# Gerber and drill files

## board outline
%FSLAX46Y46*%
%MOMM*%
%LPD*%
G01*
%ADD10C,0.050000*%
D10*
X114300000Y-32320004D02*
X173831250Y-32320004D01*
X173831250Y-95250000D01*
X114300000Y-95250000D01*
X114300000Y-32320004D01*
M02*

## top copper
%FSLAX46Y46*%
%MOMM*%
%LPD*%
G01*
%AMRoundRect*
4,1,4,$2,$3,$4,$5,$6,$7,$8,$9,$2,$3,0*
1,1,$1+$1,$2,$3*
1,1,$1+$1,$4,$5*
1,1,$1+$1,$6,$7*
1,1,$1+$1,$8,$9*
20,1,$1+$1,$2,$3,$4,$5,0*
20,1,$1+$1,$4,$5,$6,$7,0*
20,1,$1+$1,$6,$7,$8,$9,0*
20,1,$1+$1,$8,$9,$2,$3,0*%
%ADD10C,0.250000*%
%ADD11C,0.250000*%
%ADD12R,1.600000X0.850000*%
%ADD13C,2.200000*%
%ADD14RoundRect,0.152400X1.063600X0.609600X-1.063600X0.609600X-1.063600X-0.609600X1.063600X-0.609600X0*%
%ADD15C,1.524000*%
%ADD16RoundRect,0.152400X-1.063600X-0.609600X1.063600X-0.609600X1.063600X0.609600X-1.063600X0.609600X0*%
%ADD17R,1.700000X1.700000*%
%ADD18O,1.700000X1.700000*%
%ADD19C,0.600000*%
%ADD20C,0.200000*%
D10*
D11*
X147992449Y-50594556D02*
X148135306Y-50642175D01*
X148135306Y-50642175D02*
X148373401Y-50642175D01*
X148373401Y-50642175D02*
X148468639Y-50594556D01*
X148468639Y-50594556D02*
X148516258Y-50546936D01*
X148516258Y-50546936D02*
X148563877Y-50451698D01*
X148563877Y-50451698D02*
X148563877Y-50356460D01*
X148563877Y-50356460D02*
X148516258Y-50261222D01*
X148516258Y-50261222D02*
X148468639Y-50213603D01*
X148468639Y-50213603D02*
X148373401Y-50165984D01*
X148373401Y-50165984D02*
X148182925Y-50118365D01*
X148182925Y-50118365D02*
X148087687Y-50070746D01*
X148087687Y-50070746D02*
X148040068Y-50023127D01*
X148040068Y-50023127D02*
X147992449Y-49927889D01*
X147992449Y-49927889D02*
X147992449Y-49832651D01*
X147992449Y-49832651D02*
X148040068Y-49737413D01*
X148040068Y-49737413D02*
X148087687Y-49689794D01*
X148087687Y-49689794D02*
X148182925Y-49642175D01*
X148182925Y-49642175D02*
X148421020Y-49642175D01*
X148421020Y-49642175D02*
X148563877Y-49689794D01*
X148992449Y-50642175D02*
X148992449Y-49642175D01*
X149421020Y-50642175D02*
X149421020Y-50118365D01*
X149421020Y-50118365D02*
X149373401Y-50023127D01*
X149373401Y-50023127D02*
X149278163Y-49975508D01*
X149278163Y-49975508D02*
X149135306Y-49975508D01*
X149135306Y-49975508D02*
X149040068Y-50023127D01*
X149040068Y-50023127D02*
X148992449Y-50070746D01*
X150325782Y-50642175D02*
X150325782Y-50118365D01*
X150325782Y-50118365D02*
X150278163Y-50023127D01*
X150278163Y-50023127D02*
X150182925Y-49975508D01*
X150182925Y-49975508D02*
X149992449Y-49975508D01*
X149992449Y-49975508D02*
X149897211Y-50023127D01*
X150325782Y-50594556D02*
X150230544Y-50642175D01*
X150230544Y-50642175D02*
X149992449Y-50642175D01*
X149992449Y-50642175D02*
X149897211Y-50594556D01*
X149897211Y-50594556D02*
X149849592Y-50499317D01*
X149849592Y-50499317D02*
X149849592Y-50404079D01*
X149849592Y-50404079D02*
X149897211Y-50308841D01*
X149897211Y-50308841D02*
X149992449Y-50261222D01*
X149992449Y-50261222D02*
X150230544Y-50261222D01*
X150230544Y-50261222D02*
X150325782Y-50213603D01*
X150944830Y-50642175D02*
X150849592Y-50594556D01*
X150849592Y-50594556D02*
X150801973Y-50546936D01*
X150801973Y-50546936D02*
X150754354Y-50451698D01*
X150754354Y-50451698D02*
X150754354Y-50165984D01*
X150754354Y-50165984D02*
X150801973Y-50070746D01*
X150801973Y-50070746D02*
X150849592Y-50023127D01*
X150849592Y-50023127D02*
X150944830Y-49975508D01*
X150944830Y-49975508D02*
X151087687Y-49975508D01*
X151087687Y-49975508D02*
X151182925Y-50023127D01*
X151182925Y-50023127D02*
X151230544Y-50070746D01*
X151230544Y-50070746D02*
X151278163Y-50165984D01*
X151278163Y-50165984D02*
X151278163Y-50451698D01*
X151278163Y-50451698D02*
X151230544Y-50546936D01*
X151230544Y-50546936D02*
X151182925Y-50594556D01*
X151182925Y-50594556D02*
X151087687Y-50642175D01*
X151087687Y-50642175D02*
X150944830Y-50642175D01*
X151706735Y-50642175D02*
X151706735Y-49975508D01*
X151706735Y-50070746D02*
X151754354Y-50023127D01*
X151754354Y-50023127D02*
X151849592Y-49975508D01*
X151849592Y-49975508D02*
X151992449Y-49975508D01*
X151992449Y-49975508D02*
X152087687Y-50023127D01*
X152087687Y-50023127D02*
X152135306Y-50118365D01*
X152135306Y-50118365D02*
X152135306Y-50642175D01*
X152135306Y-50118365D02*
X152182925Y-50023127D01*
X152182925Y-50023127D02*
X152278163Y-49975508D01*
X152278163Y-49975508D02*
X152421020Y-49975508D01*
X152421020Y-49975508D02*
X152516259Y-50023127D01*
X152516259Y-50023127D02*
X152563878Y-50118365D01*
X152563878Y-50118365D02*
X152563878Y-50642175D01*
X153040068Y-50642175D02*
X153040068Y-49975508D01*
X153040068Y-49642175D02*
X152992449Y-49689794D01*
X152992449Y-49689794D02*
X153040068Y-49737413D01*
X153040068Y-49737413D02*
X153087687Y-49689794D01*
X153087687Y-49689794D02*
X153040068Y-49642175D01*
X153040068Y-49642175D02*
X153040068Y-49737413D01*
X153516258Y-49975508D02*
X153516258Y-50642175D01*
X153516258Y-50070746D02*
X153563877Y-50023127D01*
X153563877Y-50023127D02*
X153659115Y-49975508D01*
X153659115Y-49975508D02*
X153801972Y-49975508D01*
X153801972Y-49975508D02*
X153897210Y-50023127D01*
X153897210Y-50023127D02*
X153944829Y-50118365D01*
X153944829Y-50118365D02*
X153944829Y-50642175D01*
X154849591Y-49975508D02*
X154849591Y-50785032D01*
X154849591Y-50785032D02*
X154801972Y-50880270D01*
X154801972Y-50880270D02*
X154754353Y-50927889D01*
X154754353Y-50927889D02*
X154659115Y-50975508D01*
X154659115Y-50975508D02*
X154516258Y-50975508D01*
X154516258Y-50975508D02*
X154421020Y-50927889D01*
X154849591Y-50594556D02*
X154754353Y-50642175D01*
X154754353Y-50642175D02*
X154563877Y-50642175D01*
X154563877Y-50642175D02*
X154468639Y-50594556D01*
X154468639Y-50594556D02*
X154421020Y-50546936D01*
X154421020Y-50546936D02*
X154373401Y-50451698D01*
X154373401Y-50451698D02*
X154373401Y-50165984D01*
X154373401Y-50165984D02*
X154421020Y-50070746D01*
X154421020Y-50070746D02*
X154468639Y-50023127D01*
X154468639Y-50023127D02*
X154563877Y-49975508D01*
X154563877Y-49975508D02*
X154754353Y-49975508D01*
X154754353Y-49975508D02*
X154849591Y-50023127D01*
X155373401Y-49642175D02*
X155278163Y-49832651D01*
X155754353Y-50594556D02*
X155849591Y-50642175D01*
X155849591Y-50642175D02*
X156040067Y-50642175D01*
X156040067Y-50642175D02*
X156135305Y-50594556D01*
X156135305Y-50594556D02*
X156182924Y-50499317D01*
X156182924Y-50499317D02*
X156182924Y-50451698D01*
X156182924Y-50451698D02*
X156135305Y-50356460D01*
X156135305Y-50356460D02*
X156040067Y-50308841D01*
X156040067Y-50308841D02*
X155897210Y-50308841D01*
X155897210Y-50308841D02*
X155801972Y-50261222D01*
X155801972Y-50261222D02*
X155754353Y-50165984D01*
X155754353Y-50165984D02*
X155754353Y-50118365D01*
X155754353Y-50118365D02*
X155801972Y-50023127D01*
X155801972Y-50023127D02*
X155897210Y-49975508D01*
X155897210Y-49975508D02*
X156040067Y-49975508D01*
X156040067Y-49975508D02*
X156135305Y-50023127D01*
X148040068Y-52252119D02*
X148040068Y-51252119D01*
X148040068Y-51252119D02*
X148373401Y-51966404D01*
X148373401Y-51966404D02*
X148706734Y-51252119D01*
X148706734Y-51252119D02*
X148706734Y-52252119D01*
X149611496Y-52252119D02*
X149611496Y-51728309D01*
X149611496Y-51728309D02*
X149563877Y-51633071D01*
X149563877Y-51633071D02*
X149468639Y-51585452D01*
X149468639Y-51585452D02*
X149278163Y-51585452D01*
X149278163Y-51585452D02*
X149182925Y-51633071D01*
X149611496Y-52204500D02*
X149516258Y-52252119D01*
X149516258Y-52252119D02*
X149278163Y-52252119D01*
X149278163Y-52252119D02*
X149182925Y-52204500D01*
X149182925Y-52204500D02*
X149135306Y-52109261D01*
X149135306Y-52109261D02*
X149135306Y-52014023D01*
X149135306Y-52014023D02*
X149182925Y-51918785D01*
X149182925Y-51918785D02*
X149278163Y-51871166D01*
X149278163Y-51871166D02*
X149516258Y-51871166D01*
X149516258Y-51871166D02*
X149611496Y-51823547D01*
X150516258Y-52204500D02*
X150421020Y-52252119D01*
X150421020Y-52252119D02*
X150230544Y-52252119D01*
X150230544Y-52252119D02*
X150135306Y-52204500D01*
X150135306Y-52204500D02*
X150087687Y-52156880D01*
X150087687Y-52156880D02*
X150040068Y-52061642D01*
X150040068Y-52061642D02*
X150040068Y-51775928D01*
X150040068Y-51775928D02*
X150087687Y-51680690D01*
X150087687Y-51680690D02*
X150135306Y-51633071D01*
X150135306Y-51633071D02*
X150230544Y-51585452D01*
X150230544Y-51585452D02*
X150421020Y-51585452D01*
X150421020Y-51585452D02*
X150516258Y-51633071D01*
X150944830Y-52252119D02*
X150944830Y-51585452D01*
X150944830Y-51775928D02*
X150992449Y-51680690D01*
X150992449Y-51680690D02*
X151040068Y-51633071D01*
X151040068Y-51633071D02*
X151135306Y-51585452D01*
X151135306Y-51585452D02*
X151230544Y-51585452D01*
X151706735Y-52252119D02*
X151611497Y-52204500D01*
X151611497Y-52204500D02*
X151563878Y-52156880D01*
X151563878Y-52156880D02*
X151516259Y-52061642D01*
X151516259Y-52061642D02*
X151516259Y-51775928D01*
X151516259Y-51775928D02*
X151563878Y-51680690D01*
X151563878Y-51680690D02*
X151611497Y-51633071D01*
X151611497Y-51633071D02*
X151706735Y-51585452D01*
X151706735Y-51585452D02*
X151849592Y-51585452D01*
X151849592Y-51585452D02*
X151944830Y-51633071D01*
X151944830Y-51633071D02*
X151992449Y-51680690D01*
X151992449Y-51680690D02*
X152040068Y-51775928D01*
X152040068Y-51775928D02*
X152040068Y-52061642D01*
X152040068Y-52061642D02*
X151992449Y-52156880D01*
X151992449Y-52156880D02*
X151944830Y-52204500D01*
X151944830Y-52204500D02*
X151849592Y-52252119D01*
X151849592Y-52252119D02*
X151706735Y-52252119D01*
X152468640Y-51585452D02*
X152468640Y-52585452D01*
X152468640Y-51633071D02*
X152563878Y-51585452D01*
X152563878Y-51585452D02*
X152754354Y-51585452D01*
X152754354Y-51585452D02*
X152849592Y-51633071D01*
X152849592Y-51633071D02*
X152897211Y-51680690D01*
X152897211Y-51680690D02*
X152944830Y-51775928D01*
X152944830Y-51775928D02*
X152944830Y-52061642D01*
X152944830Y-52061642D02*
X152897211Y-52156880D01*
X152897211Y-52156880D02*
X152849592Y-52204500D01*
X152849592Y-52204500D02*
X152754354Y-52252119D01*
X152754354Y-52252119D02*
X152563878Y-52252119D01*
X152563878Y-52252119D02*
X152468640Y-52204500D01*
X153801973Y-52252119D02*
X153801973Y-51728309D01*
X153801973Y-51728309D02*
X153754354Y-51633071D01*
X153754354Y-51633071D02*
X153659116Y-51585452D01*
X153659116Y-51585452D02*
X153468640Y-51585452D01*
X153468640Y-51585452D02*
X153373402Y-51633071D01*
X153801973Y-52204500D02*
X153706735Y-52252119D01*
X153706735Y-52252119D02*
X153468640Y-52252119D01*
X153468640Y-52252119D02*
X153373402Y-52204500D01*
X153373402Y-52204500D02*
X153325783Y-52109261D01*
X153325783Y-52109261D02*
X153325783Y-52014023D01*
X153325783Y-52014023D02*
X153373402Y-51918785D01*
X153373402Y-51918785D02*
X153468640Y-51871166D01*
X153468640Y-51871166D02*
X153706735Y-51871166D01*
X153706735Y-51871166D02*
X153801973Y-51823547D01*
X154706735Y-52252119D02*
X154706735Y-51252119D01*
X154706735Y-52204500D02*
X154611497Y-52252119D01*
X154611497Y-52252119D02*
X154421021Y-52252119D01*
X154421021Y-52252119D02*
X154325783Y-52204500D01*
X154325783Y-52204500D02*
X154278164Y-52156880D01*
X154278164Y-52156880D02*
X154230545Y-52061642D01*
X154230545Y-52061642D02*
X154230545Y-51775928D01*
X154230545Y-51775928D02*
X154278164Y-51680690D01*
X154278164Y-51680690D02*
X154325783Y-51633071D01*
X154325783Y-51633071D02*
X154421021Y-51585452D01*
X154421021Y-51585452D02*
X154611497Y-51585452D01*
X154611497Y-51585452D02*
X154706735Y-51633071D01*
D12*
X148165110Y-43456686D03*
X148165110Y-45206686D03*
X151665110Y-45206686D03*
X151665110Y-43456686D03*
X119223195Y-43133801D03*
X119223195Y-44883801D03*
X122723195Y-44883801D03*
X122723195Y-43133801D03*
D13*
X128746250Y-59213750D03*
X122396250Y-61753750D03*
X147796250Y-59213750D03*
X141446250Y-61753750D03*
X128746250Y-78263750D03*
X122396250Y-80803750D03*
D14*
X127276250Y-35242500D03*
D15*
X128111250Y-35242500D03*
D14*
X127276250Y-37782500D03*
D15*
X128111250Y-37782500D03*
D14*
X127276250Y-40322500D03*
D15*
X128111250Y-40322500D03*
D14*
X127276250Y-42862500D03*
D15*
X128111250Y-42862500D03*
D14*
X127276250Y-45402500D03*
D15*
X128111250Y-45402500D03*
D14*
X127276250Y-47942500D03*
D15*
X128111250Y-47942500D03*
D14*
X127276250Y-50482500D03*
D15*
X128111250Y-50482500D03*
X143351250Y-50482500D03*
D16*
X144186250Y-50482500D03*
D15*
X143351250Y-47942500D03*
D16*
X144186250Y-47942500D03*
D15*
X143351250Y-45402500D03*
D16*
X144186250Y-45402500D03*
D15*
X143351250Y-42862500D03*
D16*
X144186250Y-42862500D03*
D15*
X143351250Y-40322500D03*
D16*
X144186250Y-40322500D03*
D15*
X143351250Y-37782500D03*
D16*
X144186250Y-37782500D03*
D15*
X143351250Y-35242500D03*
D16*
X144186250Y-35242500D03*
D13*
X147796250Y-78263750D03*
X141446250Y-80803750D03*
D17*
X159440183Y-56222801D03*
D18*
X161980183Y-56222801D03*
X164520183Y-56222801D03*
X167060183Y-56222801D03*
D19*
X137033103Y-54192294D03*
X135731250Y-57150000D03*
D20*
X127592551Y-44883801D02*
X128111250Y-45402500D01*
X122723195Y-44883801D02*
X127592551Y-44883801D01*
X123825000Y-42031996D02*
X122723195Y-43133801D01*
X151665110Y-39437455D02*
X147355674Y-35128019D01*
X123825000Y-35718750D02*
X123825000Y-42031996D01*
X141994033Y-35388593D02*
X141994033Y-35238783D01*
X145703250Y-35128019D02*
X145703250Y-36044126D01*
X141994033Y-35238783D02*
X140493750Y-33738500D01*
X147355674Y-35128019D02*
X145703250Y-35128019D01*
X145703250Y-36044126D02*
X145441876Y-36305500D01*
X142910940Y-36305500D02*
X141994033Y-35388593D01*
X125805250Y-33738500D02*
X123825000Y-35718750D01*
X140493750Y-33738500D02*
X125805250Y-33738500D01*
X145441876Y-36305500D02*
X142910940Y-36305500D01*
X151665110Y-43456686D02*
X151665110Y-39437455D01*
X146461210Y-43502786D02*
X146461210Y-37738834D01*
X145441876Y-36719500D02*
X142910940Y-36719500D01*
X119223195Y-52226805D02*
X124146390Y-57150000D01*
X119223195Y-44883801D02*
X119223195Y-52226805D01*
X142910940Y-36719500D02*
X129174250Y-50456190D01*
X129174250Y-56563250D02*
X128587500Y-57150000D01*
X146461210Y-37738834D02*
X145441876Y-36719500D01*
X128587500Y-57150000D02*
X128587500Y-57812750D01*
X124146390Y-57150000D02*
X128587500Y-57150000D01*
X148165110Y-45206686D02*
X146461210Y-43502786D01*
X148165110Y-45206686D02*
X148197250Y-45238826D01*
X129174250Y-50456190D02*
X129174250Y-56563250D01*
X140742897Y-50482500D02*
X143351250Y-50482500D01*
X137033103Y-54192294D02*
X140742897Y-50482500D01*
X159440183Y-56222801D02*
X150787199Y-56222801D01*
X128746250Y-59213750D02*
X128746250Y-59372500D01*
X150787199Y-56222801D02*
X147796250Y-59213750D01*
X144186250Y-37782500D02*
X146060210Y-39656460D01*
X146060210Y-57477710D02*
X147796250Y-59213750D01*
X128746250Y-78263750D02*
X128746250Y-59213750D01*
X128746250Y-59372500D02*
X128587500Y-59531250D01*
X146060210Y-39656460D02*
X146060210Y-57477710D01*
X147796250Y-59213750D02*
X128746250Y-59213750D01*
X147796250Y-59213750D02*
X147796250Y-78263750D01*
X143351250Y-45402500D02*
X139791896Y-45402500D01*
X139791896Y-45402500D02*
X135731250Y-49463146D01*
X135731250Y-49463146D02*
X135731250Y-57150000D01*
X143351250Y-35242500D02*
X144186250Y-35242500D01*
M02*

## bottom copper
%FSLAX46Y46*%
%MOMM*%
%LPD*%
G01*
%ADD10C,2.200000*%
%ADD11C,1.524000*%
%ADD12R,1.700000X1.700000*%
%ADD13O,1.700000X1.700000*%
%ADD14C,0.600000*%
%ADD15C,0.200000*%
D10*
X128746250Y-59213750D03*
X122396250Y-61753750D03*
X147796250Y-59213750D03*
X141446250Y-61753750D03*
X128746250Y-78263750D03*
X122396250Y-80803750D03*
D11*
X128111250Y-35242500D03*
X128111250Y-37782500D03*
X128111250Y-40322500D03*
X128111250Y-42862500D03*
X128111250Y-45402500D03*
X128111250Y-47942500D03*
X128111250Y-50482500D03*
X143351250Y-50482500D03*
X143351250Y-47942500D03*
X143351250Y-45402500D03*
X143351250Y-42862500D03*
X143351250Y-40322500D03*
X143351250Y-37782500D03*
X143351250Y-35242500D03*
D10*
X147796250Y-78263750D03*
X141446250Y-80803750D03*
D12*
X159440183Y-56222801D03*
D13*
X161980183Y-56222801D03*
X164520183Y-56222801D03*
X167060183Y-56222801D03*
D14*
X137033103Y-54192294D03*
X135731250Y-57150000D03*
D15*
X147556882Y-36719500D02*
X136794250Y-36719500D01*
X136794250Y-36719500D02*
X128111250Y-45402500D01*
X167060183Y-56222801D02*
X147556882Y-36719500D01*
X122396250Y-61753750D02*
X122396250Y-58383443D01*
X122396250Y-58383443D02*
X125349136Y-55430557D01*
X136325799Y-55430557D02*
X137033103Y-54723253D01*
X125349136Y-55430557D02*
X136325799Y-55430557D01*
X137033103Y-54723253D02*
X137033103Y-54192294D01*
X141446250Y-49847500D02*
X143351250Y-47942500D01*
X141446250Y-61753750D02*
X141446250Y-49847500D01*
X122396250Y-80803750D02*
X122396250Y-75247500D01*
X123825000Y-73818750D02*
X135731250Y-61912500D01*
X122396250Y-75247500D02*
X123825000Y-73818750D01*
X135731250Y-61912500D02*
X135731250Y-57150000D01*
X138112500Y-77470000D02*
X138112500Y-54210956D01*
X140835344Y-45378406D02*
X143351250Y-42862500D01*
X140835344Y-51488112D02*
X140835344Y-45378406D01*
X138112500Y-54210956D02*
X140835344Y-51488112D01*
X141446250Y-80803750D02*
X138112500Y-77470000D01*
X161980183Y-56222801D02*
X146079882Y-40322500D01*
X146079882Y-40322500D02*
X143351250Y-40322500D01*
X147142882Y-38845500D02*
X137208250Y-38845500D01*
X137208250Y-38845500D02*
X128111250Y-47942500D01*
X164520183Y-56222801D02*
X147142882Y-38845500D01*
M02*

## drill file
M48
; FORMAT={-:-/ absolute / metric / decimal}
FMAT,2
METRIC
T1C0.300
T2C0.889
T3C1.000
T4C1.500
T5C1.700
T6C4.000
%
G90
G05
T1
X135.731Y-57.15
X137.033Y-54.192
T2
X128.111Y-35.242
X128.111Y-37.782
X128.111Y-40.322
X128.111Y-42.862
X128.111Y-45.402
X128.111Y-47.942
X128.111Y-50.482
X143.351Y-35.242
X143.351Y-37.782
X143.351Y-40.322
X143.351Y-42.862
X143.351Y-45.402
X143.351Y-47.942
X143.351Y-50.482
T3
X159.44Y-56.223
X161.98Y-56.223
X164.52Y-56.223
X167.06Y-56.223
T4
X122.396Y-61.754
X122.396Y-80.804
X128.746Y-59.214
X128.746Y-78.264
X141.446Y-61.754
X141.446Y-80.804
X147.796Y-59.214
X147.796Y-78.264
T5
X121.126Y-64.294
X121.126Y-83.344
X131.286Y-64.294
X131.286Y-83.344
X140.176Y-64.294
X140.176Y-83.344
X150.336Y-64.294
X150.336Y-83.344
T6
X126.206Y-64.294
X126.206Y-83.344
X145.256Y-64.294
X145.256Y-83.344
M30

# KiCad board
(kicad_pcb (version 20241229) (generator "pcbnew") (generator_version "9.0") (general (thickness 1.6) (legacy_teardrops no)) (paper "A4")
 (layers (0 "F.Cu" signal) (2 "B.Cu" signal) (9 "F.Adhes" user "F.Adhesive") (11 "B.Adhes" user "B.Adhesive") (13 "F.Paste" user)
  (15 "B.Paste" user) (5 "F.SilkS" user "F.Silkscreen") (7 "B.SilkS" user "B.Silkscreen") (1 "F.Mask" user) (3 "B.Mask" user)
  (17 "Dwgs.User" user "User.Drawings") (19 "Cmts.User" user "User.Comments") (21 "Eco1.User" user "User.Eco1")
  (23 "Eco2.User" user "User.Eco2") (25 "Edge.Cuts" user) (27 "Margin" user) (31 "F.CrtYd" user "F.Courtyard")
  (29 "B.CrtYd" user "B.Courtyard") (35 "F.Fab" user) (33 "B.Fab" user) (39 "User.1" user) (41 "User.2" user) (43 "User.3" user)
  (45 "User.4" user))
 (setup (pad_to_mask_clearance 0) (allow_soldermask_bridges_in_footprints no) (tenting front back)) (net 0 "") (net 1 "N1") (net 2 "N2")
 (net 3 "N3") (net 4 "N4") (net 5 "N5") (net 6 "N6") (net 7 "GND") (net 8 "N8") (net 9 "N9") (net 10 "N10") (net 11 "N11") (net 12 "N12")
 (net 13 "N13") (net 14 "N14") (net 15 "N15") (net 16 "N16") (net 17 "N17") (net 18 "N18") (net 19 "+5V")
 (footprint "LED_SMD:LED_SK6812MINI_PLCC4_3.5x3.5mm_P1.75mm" (layer "F.Cu") (at 149.91511 44.331686)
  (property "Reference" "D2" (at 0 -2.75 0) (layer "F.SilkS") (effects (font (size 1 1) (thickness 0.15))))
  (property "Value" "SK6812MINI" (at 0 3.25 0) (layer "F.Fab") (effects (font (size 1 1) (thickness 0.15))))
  (pad "1" smd rect (at -1.75 -0.875) (size 1.6 0.85) (layers "F.Cu" "F.Mask" "F.Paste") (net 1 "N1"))
  (pad "2" smd rect (at -1.75 0.875) (size 1.6 0.85) (layers "F.Cu" "F.Mask" "F.Paste") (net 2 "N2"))
  (pad "3" smd rect (at 1.75 0.875) (size 1.6 0.85) (layers "F.Cu" "F.Mask" "F.Paste") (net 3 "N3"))
  (pad "4" smd rect (at 1.75 -0.875) (size 1.6 0.85) (layers "F.Cu" "F.Mask" "F.Paste") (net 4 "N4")))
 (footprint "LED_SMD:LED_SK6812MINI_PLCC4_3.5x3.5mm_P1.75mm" (layer "F.Cu") (at 120.973195 44.008801)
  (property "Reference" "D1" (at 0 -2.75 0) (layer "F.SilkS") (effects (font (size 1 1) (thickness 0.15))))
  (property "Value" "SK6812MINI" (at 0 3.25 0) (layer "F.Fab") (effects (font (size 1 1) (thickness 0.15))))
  (pad "1" smd rect (at -1.75 -0.875) (size 1.6 0.85) (layers "F.Cu" "F.Mask" "F.Paste") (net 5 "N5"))
  (pad "2" smd rect (at -1.75 0.875) (size 1.6 0.85) (layers "F.Cu" "F.Mask" "F.Paste") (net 2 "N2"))
  (pad "3" smd rect (at 1.75 0.875) (size 1.6 0.85) (layers "F.Cu" "F.Mask" "F.Paste") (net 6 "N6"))
  (pad "4" smd rect (at 1.75 -0.875) (size 1.6 0.85) (layers "F.Cu" "F.Mask" "F.Paste") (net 4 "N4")))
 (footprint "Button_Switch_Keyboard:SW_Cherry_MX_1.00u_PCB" (layer "F.Cu") (at 128.74625 59.21375)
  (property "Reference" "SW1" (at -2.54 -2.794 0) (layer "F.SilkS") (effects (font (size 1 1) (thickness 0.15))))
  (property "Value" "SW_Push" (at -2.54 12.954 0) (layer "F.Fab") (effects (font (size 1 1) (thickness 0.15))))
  (pad "" np_thru_hole circle (at -7.62 5.08) (size 1.7 1.7) (drill 1.7) (layers "*.Cu" "*.Mask"))
  (pad "" np_thru_hole circle (at -2.54 5.08) (size 4 4) (drill 4) (layers "*.Cu" "*.Mask"))
  (pad "" np_thru_hole circle (at 2.54 5.08) (size 1.7 1.7) (drill 1.7) (layers "*.Cu" "*.Mask"))
  (pad "1" thru_hole circle (at 0 0) (size 2.2 2.2) (drill 1.5) (layers "*.Cu" "*.Mask") (remove_unused_layers no) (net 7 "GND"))
  (pad "2" thru_hole circle (at -6.35 2.54) (size 2.2 2.2) (drill 1.5) (layers "*.Cu" "*.Mask") (remove_unused_layers no) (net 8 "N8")))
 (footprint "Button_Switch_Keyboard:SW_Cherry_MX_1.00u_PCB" (layer "F.Cu") (at 147.79625 59.21375)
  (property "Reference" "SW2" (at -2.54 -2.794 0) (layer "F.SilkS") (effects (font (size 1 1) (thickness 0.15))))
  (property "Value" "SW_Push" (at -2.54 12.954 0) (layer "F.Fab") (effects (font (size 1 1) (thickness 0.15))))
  (pad "" np_thru_hole circle (at -7.62 5.08) (size 1.7 1.7) (drill 1.7) (layers "*.Cu" "*.Mask"))
  (pad "" np_thru_hole circle (at -2.54 5.08) (size 4 4) (drill 4) (layers "*.Cu" "*.Mask"))
  (pad "" np_thru_hole circle (at 2.54 5.08) (size 1.7 1.7) (drill 1.7) (layers "*.Cu" "*.Mask"))
  (pad "1" thru_hole circle (at 0 0) (size 2.2 2.2) (drill 1.5) (layers "*.Cu" "*.Mask") (remove_unused_layers no) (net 7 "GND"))
  (pad "2" thru_hole circle (at -6.35 2.54) (size 2.2 2.2) (drill 1.5) (layers "*.Cu" "*.Mask") (remove_unused_layers no) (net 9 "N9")))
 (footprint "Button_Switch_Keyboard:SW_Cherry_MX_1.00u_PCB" (layer "F.Cu") (at 128.74625 78.26375)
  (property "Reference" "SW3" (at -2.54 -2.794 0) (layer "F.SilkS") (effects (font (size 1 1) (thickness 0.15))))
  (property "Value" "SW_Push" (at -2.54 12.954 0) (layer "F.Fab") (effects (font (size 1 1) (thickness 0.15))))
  (pad "" np_thru_hole circle (at -7.62 5.08) (size 1.7 1.7) (drill 1.7) (layers "*.Cu" "*.Mask"))
  (pad "" np_thru_hole circle (at -2.54 5.08) (size 4 4) (drill 4) (layers "*.Cu" "*.Mask"))
  (pad "" np_thru_hole circle (at 2.54 5.08) (size 1.7 1.7) (drill 1.7) (layers "*.Cu" "*.Mask"))
  (pad "1" thru_hole circle (at 0 0) (size 2.2 2.2) (drill 1.5) (layers "*.Cu" "*.Mask") (remove_unused_layers no) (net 7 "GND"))
  (pad "2" thru_hole circle (at -6.35 2.54) (size 2.2 2.2) (drill 1.5) (layers "*.Cu" "*.Mask") (remove_unused_layers no) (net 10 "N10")))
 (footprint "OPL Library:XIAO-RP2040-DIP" (layer "F.Cu") (at 135.73125 42.8625)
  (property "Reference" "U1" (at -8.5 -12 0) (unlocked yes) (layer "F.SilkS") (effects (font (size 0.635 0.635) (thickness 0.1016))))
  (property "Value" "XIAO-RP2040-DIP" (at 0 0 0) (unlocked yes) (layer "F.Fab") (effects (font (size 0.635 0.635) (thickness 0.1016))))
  (pad "1" smd roundrect (at -8.455 -7.62 180) (size 2.432 1.524) (layers "F.Cu" "F.Mask") (roundrect_rratio 0.1) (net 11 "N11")
   (thermal_bridge_angle 45))
  (pad "1" thru_hole circle (at -7.62 -7.62 180) (size 1.524 1.524) (drill 0.889) (layers "*.Cu" "*.Mask") (remove_unused_layers no)
   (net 11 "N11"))
  (pad "2" smd roundrect (at -8.455 -5.08 180) (size 2.432 1.524) (layers "F.Cu" "F.Mask") (roundrect_rratio 0.1) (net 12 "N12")
   (thermal_bridge_angle 45))
  (pad "2" thru_hole circle (at -7.62 -5.08 180) (size 1.524 1.524) (drill 0.889) (layers "*.Cu" "*.Mask") (remove_unused_layers no)
   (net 12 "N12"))
  (pad "3" smd roundrect (at -8.455 -2.54 180) (size 2.432 1.524) (layers "F.Cu" "F.Mask") (roundrect_rratio 0.1) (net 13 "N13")
   (thermal_bridge_angle 45))
  (pad "3" thru_hole circle (at -7.62 -2.54 180) (size 1.524 1.524) (drill 0.889) (layers "*.Cu" "*.Mask") (remove_unused_layers no)
   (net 13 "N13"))
  (pad "4" smd roundrect (at -8.455 0 180) (size 2.432 1.524) (layers "F.Cu" "F.Mask") (roundrect_rratio 0.1) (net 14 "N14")
   (thermal_bridge_angle 45))
  (pad "4" thru_hole circle (at -7.62 0 180) (size 1.524 1.524) (drill 0.889) (layers "*.Cu" "*.Mask") (remove_unused_layers no)
   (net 14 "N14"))
  (pad "5" smd roundrect (at -8.455 2.54 180) (size 2.432 1.524) (layers "F.Cu" "F.Mask") (roundrect_rratio 0.1) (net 6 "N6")
   (thermal_bridge_angle 45))
  (pad "5" thru_hole circle (at -7.62 2.54 180) (size 1.524 1.524) (drill 0.889) (layers "*.Cu" "*.Mask") (remove_unused_layers no)
   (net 6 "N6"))
  (pad "6" smd roundrect (at -8.455 5.08 180) (size 2.432 1.524) (layers "F.Cu" "F.Mask") (roundrect_rratio 0.1) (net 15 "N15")
   (thermal_bridge_angle 45))
  (pad "6" thru_hole circle (at -7.62 5.08 180) (size 1.524 1.524) (drill 0.889) (layers "*.Cu" "*.Mask") (remove_unused_layers no)
   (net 15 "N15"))
  (pad "7" smd roundrect (at -8.455 7.62 180) (size 2.432 1.524) (layers "F.Cu" "F.Mask") (roundrect_rratio 0.1) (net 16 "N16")
   (thermal_bridge_angle 45))
  (pad "7" thru_hole circle (at -7.62 7.62 180) (size 1.524 1.524) (drill 0.889) (layers "*.Cu" "*.Mask") (remove_unused_layers no)
   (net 16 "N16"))
  (pad "8" thru_hole circle (at 7.62 7.62) (size 1.524 1.524) (drill 0.889) (layers "*.Cu" "*.Mask") (remove_unused_layers no) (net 8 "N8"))
  (pad "8" smd roundrect (at 8.455 7.62) (size 2.432 1.524) (layers "F.Cu" "F.Mask") (roundrect_rratio 0.1) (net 8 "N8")
   (thermal_bridge_angle 45))
  (pad "9" thru_hole circle (at 7.62 5.08) (size 1.524 1.524) (drill 0.889) (layers "*.Cu" "*.Mask") (remove_unused_layers no) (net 9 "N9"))
  (pad "9" smd roundrect (at 8.455 5.08) (size 2.432 1.524) (layers "F.Cu" "F.Mask") (roundrect_rratio 0.1) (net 9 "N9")
   (thermal_bridge_angle 45))
  (pad "10" thru_hole circle (at 7.62 2.54) (size 1.524 1.524) (drill 0.889) (layers "*.Cu" "*.Mask") (remove_unused_layers no)
   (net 10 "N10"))
  (pad "10" smd roundrect (at 8.455 2.54) (size 2.432 1.524) (layers "F.Cu" "F.Mask") (roundrect_rratio 0.1) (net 10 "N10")
   (thermal_bridge_angle 45))
  (pad "11" thru_hole circle (at 7.62 0) (size 1.524 1.524) (drill 0.889) (layers "*.Cu" "*.Mask") (remove_unused_layers no) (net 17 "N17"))
  (pad "11" smd roundrect (at 8.455 0) (size 2.432 1.524) (layers "F.Cu" "F.Mask") (roundrect_rratio 0.1) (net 17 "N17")
   (thermal_bridge_angle 45))
  (pad "12" thru_hole circle (at 7.62 -2.54) (size 1.524 1.524) (drill 0.889) (layers "*.Cu" "*.Mask") (remove_unused_layers no)
   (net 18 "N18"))
  (pad "12" smd roundrect (at 8.455 -2.54) (size 2.432 1.524) (layers "F.Cu" "F.Mask") (roundrect_rratio 0.1) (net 18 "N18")
   (thermal_bridge_angle 45))
  (pad "13" thru_hole circle (at 7.62 -5.08) (size 1.524 1.524) (drill 0.889) (layers "*.Cu" "*.Mask") (remove_unused_layers no)
   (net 7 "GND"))
  (pad "13" smd roundrect (at 8.455 -5.08) (size 2.432 1.524) (layers "F.Cu" "F.Mask") (roundrect_rratio 0.1) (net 7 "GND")
   (thermal_bridge_angle 45))
  (pad "14" thru_hole circle (at 7.62 -7.62) (size 1.524 1.524) (drill 0.889) (layers "*.Cu" "*.Mask") (remove_unused_layers no)
   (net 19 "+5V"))
  (pad "14" smd roundrect (at 8.455 -7.62) (size 2.432 1.524) (layers "F.Cu" "F.Mask") (roundrect_rratio 0.1) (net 19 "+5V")
   (thermal_bridge_angle 45)))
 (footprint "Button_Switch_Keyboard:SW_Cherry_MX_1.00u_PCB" (layer "F.Cu") (at 147.79625 78.26375)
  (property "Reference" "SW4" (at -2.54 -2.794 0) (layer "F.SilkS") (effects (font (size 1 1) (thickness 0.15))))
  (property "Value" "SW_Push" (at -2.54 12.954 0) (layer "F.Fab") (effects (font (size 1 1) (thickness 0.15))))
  (pad "" np_thru_hole circle (at -7.62 5.08) (size 1.7 1.7) (drill 1.7) (layers "*.Cu" "*.Mask"))
  (pad "" np_thru_hole circle (at -2.54 5.08) (size 4 4) (drill 4) (layers "*.Cu" "*.Mask"))
  (pad "" np_thru_hole circle (at 2.54 5.08) (size 1.7 1.7) (drill 1.7) (layers "*.Cu" "*.Mask"))
  (pad "1" thru_hole circle (at 0 0) (size 2.2 2.2) (drill 1.5) (layers "*.Cu" "*.Mask") (remove_unused_layers no) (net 7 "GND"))
  (pad "2" thru_hole circle (at -6.35 2.54) (size 2.2 2.2) (drill 1.5) (layers "*.Cu" "*.Mask") (remove_unused_layers no) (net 17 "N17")))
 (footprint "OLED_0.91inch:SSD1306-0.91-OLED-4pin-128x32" (layer "F.Cu") (at 157.250183 92.722801 90)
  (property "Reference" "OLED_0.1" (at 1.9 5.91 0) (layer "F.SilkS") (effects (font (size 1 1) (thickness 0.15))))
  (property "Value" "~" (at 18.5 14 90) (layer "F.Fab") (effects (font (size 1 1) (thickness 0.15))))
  (pad "1" thru_hole rect (at 36.5 2.19 90) (size 1.7 1.7) (drill 1) (layers "*.Cu" "*.Mask") (remove_unused_layers no) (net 7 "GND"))
  (pad "2" thru_hole oval (at 36.5 4.73 90) (size 1.7 1.7) (drill 1) (layers "*.Cu" "*.Mask") (remove_unused_layers no) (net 18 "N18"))
  (pad "3" thru_hole oval (at 36.5 7.27 90) (size 1.7 1.7) (drill 1) (layers "*.Cu" "*.Mask") (remove_unused_layers no) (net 15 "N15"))
  (pad "4" thru_hole oval (at 36.5 9.81 90) (size 1.7 1.7) (drill 1) (layers "*.Cu" "*.Mask") (remove_unused_layers no) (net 6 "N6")))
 (gr_rect (start 114.3 32.320004) (end 173.83125 95.25) (stroke (width 0.05) (type default)) (fill no) (layer "Edge.Cuts"))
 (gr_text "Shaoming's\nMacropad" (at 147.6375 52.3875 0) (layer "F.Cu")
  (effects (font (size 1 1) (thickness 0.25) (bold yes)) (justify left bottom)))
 (segment (start 127.592551 44.883801) (end 128.11125 45.4025) (width 0.2) (layer "F.Cu") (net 6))
 (segment (start 122.723195 44.883801) (end 127.592551 44.883801) (width 0.2) (layer "F.Cu") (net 6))
 (segment (start 147.556882 36.7195) (end 136.79425 36.7195) (width 0.2) (layer "B.Cu") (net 6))
 (segment (start 136.79425 36.7195) (end 128.11125 45.4025) (width 0.2) (layer "B.Cu") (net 6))
 (segment (start 167.060183 56.222801) (end 147.556882 36.7195) (width 0.2) (layer "B.Cu") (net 6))
 (segment (start 123.825 42.031996) (end 122.723195 43.133801) (width 0.2) (layer "F.Cu") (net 4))
 (segment (start 151.66511 39.437455) (end 147.355674 35.128019) (width 0.2) (layer "F.Cu") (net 4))
 (segment (start 123.825 35.71875) (end 123.825 42.031996) (width 0.2) (layer "F.Cu") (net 4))
 (segment (start 141.994033 35.388593) (end 141.994033 35.238783) (width 0.2) (layer "F.Cu") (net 4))
 (segment (start 145.70325 35.128019) (end 145.70325 36.044126) (width 0.2) (layer "F.Cu") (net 4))
 (segment (start 141.994033 35.238783) (end 140.49375 33.7385) (width 0.2) (layer "F.Cu") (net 4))
 (segment (start 147.355674 35.128019) (end 145.70325 35.128019) (width 0.2) (layer "F.Cu") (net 4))
 (segment (start 145.70325 36.044126) (end 145.441876 36.3055) (width 0.2) (layer "F.Cu") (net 4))
 (segment (start 142.91094 36.3055) (end 141.994033 35.388593) (width 0.2) (layer "F.Cu") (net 4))
 (segment (start 125.80525 33.7385) (end 123.825 35.71875) (width 0.2) (layer "F.Cu") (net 4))
 (segment (start 140.49375 33.7385) (end 125.80525 33.7385) (width 0.2) (layer "F.Cu") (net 4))
 (segment (start 145.441876 36.3055) (end 142.91094 36.3055) (width 0.2) (layer "F.Cu") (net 4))
 (segment (start 151.66511 43.456686) (end 151.66511 39.437455) (width 0.2) (layer "F.Cu") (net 4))
 (segment (start 146.46121 43.502786) (end 146.46121 37.738834) (width 0.2) (layer "F.Cu") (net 2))
 (segment (start 145.441876 36.7195) (end 142.91094 36.7195) (width 0.2) (layer "F.Cu") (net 2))
 (segment (start 119.223195 52.226805) (end 124.14639 57.15) (width 0.2) (layer "F.Cu") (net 2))
 (segment (start 119.223195 44.883801) (end 119.223195 52.226805) (width 0.2) (layer "F.Cu") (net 2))
 (segment (start 142.91094 36.7195) (end 129.17425 50.45619) (width 0.2) (layer "F.Cu") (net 2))
 (segment (start 129.17425 56.56325) (end 128.5875 57.15) (width 0.2) (layer "F.Cu") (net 2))
 (segment (start 146.46121 37.738834) (end 145.441876 36.7195) (width 0.2) (layer "F.Cu") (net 2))
 (segment (start 128.5875 57.15) (end 128.5875 57.81275) (width 0.2) (layer "F.Cu") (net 2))
 (segment (start 124.14639 57.15) (end 128.5875 57.15) (width 0.2) (layer "F.Cu") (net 2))
 (segment (start 148.16511 45.206686) (end 146.46121 43.502786) (width 0.2) (layer "F.Cu") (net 2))
 (segment (start 148.16511 45.206686) (end 148.19725 45.238826) (width 0.2) (layer "F.Cu") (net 2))
 (segment (start 129.17425 50.45619) (end 129.17425 56.56325) (width 0.2) (layer "F.Cu") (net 2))
 (segment (start 140.742897 50.4825) (end 143.35125 50.4825) (width 0.2) (layer "F.Cu") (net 8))
 (segment (start 137.033103 54.192294) (end 140.742897 50.4825) (width 0.2) (layer "F.Cu") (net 8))
 (via (at 137.033103 54.192294) (size 0.6) (drill 0.3) (layers "F.Cu" "B.Cu") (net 8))
 (segment (start 122.39625 61.75375) (end 122.39625 58.383443) (width 0.2) (layer "B.Cu") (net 8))
 (segment (start 122.39625 58.383443) (end 125.349136 55.430557) (width 0.2) (layer "B.Cu") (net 8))
 (segment (start 136.325799 55.430557) (end 137.033103 54.723253) (width 0.2) (layer "B.Cu") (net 8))
 (segment (start 125.349136 55.430557) (end 136.325799 55.430557) (width 0.2) (layer "B.Cu") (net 8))
 (segment (start 137.033103 54.723253) (end 137.033103 54.192294) (width 0.2) (layer "B.Cu") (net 8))
 (segment (start 159.440183 56.222801) (end 150.787199 56.222801) (width 0.2) (layer "F.Cu") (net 7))
 (segment (start 128.74625 59.21375) (end 128.74625 59.3725) (width 0.2) (layer "F.Cu") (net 7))
 (segment (start 150.787199 56.222801) (end 147.79625 59.21375) (width 0.2) (layer "F.Cu") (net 7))
 (segment (start 144.18625 37.7825) (end 146.06021 39.65646) (width 0.2) (layer "F.Cu") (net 7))
 (segment (start 146.06021 57.47771) (end 147.79625 59.21375) (width 0.2) (layer "F.Cu") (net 7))
 (segment (start 128.74625 78.26375) (end 128.74625 59.21375) (width 0.2) (layer "F.Cu") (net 7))
 (segment (start 128.74625 59.3725) (end 128.5875 59.53125) (width 0.2) (layer "F.Cu") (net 7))
 (segment (start 146.06021 39.65646) (end 146.06021 57.47771) (width 0.2) (layer "F.Cu") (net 7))
 (segment (start 147.79625 59.21375) (end 128.74625 59.21375) (width 0.2) (layer "F.Cu") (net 7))
 (segment (start 147.79625 59.21375) (end 147.79625 78.26375) (width 0.2) (layer "F.Cu") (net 7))
 (segment (start 141.44625 49.8475) (end 143.35125 47.9425) (width 0.2) (layer "B.Cu") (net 9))
 (segment (start 141.44625 61.75375) (end 141.44625 49.8475) (width 0.2) (layer "B.Cu") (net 9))
 (segment (start 143.35125 45.4025) (end 139.791896 45.4025) (width 0.2) (layer "F.Cu") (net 10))
 (segment (start 139.791896 45.4025) (end 135.73125 49.463146) (width 0.2) (layer "F.Cu") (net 10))
 (segment (start 135.73125 49.463146) (end 135.73125 57.15) (width 0.2) (layer "F.Cu") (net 10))
 (via (at 135.73125 57.15) (size 0.6) (drill 0.3) (layers "F.Cu" "B.Cu") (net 10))
 (segment (start 122.39625 80.80375) (end 122.39625 75.2475) (width 0.2) (layer "B.Cu") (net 10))
 (segment (start 123.825 73.81875) (end 135.73125 61.9125) (width 0.2) (layer "B.Cu") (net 10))
 (segment (start 122.39625 75.2475) (end 123.825 73.81875) (width 0.2) (layer "B.Cu") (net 10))
 (segment (start 135.73125 61.9125) (end 135.73125 57.15) (width 0.2) (layer "B.Cu") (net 10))
 (segment (start 138.1125 77.47) (end 138.1125 54.210956) (width 0.2) (layer "B.Cu") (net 17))
 (segment (start 140.835344 45.378406) (end 143.35125 42.8625) (width 0.2) (layer "B.Cu") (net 17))
 (segment (start 140.835344 51.488112) (end 140.835344 45.378406) (width 0.2) (layer "B.Cu") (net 17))
 (segment (start 138.1125 54.210956) (end 140.835344 51.488112) (width 0.2) (layer "B.Cu") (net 17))
 (segment (start 141.44625 80.80375) (end 138.1125 77.47) (width 0.2) (layer "B.Cu") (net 17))
 (segment (start 161.980183 56.222801) (end 146.079882 40.3225) (width 0.2) (layer "B.Cu") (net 18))
 (segment (start 146.079882 40.3225) (end 143.35125 40.3225) (width 0.2) (layer "B.Cu") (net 18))
 (segment (start 143.35125 35.2425) (end 144.18625 35.2425) (width 0.2) (layer "F.Cu") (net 19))
 (segment (start 147.142882 38.8455) (end 137.20825 38.8455) (width 0.2) (layer "B.Cu") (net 15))
 (segment (start 137.20825 38.8455) (end 128.11125 47.9425) (width 0.2) (layer "B.Cu") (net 15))
 (segment (start 164.520183 56.222801) (end 147.142882 38.8455) (width 0.2) (layer "B.Cu") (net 15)))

